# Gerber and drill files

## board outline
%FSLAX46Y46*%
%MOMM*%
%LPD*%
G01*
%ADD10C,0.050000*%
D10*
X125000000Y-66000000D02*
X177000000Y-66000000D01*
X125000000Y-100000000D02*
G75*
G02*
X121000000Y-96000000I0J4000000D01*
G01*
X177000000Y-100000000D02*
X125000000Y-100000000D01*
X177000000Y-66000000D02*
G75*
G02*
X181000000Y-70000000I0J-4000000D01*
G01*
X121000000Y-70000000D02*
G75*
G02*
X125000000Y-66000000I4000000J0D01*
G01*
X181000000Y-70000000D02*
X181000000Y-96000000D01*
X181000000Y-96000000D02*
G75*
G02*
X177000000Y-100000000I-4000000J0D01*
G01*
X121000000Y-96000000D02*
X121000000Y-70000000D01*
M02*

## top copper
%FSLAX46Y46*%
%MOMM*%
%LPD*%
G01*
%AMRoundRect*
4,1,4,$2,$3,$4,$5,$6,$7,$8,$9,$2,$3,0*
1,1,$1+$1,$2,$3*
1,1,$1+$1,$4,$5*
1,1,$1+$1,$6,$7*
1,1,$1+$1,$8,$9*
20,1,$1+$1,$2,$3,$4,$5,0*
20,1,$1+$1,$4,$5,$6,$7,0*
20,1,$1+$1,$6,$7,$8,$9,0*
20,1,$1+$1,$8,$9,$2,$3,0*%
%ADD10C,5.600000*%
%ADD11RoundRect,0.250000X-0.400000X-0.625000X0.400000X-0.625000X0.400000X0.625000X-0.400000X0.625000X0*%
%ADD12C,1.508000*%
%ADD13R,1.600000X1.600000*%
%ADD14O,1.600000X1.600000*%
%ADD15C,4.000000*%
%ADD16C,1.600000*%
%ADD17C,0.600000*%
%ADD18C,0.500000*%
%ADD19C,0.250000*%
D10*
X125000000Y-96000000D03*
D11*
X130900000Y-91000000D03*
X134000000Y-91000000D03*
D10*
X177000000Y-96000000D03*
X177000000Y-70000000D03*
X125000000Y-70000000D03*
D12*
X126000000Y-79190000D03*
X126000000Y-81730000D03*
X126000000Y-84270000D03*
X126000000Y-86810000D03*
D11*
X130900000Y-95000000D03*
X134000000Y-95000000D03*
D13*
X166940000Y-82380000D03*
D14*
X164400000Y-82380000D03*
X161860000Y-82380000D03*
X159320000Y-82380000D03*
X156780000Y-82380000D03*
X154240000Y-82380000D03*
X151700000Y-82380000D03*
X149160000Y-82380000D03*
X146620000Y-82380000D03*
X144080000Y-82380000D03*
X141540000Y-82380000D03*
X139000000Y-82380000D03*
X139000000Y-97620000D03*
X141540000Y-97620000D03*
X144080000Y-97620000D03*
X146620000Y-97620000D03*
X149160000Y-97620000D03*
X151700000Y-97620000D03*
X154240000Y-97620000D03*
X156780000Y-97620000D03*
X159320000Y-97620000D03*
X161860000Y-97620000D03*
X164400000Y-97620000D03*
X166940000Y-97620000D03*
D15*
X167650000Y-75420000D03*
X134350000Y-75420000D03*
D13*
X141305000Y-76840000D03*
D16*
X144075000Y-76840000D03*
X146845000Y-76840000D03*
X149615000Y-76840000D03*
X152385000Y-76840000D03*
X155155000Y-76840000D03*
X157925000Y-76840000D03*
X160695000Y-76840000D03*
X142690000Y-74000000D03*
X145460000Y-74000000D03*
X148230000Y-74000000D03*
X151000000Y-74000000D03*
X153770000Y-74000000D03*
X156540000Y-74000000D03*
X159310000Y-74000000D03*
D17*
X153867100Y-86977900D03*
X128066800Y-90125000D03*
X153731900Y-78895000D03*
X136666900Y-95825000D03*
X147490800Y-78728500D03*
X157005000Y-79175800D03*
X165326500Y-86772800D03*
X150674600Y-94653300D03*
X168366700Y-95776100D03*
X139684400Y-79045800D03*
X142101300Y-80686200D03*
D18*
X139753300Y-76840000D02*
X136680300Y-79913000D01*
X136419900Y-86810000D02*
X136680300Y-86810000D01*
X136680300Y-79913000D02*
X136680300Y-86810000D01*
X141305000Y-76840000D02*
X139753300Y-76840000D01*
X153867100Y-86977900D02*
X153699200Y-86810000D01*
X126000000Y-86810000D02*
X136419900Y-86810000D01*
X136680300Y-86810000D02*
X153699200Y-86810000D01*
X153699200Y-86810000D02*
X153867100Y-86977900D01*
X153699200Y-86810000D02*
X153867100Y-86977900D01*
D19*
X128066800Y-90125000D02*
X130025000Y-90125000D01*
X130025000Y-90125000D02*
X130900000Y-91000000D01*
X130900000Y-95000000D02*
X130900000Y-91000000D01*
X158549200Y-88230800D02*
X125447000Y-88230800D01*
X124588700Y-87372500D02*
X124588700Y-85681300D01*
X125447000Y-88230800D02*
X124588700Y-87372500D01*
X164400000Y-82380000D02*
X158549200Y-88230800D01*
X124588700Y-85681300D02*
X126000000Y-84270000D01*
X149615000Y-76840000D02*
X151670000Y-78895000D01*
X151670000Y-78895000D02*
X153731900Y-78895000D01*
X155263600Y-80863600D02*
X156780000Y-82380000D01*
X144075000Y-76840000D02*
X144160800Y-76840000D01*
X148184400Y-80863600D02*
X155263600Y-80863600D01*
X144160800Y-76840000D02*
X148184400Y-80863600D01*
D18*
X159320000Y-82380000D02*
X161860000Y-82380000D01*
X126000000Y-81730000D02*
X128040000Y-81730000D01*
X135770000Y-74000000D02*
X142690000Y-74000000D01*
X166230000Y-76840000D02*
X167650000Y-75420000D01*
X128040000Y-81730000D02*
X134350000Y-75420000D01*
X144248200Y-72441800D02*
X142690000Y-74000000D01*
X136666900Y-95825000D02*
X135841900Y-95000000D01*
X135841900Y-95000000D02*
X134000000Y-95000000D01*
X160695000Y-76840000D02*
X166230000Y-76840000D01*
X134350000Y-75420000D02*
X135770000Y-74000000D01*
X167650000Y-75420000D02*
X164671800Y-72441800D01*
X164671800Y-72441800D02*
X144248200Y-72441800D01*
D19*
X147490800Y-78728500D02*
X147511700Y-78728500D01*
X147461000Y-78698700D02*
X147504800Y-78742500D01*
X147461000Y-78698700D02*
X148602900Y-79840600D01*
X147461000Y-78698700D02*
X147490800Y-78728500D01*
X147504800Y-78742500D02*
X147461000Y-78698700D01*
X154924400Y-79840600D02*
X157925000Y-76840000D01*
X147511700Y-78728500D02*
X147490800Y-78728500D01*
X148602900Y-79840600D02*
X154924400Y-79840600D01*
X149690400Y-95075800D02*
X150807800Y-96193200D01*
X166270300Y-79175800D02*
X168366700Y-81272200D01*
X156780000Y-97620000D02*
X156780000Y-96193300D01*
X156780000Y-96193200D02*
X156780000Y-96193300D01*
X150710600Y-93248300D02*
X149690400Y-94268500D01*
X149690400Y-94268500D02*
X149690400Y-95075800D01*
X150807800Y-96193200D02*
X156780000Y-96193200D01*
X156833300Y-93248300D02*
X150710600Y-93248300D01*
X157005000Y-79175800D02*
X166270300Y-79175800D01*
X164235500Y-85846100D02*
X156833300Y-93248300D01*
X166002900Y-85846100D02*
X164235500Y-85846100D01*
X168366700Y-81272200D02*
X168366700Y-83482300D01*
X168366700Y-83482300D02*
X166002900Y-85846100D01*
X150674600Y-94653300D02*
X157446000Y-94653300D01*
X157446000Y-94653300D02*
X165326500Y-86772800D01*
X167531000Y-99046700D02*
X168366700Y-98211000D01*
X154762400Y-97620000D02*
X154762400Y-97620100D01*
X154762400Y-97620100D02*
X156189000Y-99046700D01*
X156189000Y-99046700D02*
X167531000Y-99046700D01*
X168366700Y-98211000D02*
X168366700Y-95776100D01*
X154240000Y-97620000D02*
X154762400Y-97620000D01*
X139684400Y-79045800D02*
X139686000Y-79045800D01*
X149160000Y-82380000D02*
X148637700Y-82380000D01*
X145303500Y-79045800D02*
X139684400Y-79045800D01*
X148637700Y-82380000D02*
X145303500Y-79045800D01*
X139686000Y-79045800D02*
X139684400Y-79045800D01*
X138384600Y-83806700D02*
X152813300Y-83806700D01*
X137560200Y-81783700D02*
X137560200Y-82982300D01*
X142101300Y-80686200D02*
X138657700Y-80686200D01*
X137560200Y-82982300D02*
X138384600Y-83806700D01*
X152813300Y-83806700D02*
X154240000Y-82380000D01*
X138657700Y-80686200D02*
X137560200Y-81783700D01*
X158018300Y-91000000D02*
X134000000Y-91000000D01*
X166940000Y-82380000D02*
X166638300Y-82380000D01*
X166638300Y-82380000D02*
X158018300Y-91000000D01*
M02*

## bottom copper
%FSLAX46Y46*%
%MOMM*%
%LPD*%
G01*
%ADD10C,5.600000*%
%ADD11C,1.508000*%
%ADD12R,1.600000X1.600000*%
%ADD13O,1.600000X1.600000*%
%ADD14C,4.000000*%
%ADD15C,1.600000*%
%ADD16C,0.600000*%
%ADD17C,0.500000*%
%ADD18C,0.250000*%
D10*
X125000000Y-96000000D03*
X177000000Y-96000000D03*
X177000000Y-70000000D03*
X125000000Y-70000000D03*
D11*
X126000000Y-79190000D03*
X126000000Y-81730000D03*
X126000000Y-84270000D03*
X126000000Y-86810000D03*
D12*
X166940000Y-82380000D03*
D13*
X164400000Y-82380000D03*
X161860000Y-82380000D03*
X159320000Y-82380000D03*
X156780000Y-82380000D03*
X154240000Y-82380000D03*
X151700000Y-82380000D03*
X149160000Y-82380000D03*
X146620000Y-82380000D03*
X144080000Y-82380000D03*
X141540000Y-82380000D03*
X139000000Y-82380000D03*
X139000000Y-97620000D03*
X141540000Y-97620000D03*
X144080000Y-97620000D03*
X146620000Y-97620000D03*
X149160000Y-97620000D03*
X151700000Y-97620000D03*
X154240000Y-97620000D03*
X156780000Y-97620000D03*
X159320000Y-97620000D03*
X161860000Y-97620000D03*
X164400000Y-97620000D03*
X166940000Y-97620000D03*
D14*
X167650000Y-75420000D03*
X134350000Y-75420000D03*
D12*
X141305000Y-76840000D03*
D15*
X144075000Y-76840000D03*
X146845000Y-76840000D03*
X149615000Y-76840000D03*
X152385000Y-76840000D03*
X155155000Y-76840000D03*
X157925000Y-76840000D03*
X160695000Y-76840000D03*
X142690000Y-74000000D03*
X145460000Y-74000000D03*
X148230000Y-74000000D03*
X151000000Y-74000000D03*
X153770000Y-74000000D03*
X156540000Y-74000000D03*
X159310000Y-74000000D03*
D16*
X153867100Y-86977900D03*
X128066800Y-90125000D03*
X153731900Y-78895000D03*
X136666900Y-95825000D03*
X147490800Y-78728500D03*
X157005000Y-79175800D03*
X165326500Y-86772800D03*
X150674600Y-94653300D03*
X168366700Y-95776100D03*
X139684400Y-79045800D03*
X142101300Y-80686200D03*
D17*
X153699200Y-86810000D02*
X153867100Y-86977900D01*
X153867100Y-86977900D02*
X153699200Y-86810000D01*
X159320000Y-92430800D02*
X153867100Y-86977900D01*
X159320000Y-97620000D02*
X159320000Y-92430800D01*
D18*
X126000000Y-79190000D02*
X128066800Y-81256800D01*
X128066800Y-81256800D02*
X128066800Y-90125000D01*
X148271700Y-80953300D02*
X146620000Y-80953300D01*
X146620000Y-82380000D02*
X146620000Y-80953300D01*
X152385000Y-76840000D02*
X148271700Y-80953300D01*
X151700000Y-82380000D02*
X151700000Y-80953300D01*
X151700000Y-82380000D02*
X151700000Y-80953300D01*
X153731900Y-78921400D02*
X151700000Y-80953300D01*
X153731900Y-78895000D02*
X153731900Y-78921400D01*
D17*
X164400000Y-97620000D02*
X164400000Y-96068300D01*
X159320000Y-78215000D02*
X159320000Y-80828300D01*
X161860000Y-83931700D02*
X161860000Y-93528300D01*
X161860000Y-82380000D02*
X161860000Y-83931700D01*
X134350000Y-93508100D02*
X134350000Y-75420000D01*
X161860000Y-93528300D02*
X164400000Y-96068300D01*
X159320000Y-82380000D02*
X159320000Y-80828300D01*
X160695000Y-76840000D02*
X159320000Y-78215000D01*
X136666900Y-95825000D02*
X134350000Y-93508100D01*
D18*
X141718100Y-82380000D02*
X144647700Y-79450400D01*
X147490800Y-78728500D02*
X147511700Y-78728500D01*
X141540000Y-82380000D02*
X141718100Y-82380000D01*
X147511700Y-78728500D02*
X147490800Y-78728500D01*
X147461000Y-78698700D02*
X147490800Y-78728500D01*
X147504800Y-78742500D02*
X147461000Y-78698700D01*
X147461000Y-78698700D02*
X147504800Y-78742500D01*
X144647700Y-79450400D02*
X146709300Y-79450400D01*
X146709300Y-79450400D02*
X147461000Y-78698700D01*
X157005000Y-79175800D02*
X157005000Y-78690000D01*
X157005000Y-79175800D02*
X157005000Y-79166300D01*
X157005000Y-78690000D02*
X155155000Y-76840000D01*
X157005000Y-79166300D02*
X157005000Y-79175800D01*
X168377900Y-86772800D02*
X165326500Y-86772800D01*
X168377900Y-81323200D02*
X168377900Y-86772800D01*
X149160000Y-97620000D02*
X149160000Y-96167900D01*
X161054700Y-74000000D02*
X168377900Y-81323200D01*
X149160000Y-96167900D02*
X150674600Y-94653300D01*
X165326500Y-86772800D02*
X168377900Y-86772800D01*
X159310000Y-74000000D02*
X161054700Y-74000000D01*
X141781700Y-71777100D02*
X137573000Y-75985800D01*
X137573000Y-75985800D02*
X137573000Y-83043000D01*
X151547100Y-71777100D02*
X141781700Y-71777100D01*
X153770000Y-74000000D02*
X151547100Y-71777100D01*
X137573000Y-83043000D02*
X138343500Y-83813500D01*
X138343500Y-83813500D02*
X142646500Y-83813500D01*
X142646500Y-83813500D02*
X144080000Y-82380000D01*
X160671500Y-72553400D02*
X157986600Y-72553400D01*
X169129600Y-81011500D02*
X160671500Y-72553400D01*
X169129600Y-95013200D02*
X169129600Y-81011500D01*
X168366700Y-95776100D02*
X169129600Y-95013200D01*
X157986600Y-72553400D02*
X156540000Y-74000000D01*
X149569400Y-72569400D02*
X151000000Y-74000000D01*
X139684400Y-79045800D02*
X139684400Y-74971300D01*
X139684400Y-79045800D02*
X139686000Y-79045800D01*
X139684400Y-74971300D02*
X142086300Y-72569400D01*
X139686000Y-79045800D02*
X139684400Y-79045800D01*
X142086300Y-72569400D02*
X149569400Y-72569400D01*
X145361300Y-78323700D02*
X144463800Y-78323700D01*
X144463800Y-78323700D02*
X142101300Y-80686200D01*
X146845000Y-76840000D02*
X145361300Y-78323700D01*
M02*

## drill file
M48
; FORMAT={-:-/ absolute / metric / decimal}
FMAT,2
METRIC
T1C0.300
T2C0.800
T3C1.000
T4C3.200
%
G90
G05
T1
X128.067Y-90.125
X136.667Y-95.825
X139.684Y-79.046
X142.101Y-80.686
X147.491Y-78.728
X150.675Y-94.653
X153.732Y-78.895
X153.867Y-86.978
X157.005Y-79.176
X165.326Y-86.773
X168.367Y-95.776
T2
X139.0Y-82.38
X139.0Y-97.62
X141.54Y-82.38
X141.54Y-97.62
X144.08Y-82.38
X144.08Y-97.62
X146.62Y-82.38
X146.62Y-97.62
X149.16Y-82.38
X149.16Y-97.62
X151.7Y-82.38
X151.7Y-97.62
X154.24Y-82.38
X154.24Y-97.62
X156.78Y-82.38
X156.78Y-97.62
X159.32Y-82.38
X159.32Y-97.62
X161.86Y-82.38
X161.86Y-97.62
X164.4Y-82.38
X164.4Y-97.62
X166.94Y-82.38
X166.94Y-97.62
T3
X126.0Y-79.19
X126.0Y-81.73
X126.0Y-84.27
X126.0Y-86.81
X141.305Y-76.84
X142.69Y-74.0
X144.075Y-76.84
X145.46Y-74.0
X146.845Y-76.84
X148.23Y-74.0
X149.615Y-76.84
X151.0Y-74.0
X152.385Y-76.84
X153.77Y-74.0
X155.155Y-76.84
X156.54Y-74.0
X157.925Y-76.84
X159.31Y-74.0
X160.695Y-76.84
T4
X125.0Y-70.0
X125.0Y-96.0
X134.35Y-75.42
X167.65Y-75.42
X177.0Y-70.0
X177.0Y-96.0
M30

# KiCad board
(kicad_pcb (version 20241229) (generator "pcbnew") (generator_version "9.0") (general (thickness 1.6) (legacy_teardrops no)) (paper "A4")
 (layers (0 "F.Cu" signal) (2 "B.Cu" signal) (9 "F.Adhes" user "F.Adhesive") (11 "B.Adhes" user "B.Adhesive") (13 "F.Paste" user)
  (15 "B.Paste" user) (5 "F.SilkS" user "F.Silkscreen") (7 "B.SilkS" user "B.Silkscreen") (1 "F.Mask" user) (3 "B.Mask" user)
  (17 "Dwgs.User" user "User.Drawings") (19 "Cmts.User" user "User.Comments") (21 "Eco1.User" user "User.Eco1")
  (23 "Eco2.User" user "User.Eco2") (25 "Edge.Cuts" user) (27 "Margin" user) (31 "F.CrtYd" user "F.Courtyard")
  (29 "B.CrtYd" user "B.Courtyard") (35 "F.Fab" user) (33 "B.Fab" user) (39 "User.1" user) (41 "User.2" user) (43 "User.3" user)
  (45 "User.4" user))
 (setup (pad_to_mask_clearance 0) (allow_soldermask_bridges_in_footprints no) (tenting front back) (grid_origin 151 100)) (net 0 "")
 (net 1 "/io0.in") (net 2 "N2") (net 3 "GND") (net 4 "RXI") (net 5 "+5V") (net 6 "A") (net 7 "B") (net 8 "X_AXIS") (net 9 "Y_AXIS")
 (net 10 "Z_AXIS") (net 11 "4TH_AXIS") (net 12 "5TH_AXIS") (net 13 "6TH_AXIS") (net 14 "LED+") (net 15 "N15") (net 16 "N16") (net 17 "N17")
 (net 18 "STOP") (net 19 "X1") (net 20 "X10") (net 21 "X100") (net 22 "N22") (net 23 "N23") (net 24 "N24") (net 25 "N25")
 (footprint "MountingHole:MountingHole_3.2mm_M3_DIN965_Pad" (layer "F.Cu") (at 125 96)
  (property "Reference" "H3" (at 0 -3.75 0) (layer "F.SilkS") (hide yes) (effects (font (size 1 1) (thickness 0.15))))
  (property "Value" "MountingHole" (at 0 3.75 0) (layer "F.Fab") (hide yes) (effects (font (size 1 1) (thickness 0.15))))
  (pad "1" thru_hole circle (at 0 0) (size 5.6 5.6) (drill 3.2) (layers "*.Cu" "*.Mask") (remove_unused_layers no) (zone_connect 2)))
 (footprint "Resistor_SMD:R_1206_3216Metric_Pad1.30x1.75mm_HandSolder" (layer "F.Cu") (at 132.45 91)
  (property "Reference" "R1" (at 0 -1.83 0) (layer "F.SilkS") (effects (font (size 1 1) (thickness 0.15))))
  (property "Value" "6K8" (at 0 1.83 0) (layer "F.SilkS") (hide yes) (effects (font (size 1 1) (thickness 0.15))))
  (pad "1" smd roundrect (at -1.55 0) (size 1.3 1.75) (layers "F.Cu" "F.Mask" "F.Paste") (roundrect_rratio 0.192308) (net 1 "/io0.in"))
  (pad "2" smd roundrect (at 1.55 0) (size 1.3 1.75) (layers "F.Cu" "F.Mask" "F.Paste") (roundrect_rratio 0.192308) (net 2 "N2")))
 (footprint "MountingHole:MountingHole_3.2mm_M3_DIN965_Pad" (layer "F.Cu") (at 177 96)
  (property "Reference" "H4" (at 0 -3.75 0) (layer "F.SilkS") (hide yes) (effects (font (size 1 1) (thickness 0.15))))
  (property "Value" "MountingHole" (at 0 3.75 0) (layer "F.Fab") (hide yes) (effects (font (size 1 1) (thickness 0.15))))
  (pad "1" thru_hole circle (at 0 0) (size 5.6 5.6) (drill 3.2) (layers "*.Cu" "*.Mask") (remove_unused_layers no) (zone_connect 2)))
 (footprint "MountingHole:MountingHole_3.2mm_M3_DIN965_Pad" (layer "F.Cu") (at 177 70)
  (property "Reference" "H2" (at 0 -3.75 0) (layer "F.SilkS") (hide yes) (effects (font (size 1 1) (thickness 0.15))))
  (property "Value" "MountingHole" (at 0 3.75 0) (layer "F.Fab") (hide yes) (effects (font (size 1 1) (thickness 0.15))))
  (pad "1" thru_hole circle (at 0 0) (size 5.6 5.6) (drill 3.2) (layers "*.Cu" "*.Mask") (remove_unused_layers no) (zone_connect 2)))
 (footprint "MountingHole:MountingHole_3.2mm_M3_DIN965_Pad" (layer "F.Cu") (at 125 70)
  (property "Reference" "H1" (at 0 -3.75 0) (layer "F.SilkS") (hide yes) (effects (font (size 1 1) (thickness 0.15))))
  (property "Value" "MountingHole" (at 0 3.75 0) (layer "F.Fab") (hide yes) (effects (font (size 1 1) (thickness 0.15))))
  (pad "1" thru_hole circle (at 0 0) (size 5.6 5.6) (drill 3.2) (layers "*.Cu" "*.Mask") (remove_unused_layers no) (zone_connect 2)))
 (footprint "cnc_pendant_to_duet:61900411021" (layer "F.Cu") (at 122.65 83 -90)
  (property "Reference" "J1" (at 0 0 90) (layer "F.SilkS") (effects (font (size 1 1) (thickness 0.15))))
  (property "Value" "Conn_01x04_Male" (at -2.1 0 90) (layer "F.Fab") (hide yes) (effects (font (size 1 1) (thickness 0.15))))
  (pad "1" thru_hole circle (at -3.81 -3.35 270) (size 1.508 1.508) (drill 1) (layers "*.Cu" "*.Mask") (remove_unused_layers no)
   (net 1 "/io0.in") (solder_mask_margin 0.102))
  (pad "2" thru_hole circle (at -1.27 -3.35 270) (size 1.508 1.508) (drill 1) (layers "*.Cu" "*.Mask") (remove_unused_layers no)
   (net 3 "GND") (solder_mask_margin 0.102))
  (pad "3" thru_hole circle (at 1.27 -3.35 270) (size 1.508 1.508) (drill 1) (layers "*.Cu" "*.Mask") (remove_unused_layers no)
   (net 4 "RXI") (solder_mask_margin 0.102))
  (pad "4" thru_hole circle (at 3.81 -3.35 270) (size 1.508 1.508) (drill 1) (layers "*.Cu" "*.Mask") (remove_unused_layers no)
   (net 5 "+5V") (solder_mask_margin 0.102)))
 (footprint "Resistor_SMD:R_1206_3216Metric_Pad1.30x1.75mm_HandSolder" (layer "F.Cu") (at 132.45 95)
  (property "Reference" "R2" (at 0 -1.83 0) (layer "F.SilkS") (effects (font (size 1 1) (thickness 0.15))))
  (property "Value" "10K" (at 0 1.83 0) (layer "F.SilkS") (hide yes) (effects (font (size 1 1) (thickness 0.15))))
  (pad "1" smd roundrect (at -1.55 0) (size 1.3 1.75) (layers "F.Cu" "F.Mask" "F.Paste") (roundrect_rratio 0.192308) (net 1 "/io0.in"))
  (pad "2" smd roundrect (at 1.55 0) (size 1.3 1.75) (layers "F.Cu" "F.Mask" "F.Paste") (roundrect_rratio 0.192308) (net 3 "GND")))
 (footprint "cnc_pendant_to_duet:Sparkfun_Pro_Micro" (layer "F.Cu") (at 139 97.62 90)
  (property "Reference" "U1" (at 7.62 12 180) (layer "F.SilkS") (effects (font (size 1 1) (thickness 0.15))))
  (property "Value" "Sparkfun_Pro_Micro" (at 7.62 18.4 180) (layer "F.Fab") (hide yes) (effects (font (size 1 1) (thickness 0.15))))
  (pad "1" thru_hole rect (at 15.24 27.94 90) (size 1.6 1.6) (drill 0.8) (layers "*.Cu" "*.Mask") (remove_unused_layers no) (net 2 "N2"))
  (pad "2" thru_hole oval (at 15.24 25.4 90) (size 1.6 1.6) (drill 0.8) (layers "*.Cu" "*.Mask") (remove_unused_layers no) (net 4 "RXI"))
  (pad "3" thru_hole oval (at 15.24 22.86 90) (size 1.6 1.6) (drill 0.8) (layers "*.Cu" "*.Mask") (remove_unused_layers no) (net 3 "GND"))
  (pad "4" thru_hole oval (at 15.24 20.32 90) (size 1.6 1.6) (drill 0.8) (layers "*.Cu" "*.Mask") (remove_unused_layers no) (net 3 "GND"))
  (pad "5" thru_hole oval (at 15.24 17.78 90) (size 1.6 1.6) (drill 0.8) (layers "*.Cu" "*.Mask") (remove_unused_layers no) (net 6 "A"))
  (pad "6" thru_hole oval (at 15.24 15.24 90) (size 1.6 1.6) (drill 0.8) (layers "*.Cu" "*.Mask") (remove_unused_layers no) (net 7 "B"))
  (pad "7" thru_hole oval (at 15.24 12.7 90) (size 1.6 1.6) (drill 0.8) (layers "*.Cu" "*.Mask") (remove_unused_layers no) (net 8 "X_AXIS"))
  (pad "8" thru_hole oval (at 15.24 10.16 90) (size 1.6 1.6) (drill 0.8) (layers "*.Cu" "*.Mask") (remove_unused_layers no) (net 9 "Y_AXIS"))
  (pad "9" thru_hole oval (at 15.24 7.62 90) (size 1.6 1.6) (drill 0.8) (layers "*.Cu" "*.Mask") (remove_unused_layers no) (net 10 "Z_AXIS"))
  (pad "10" thru_hole oval (at 15.24 5.08 90) (size 1.6 1.6) (drill 0.8) (layers "*.Cu" "*.Mask") (remove_unused_layers no)
   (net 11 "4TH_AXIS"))
  (pad "11" thru_hole oval (at 15.24 2.54 90) (size 1.6 1.6) (drill 0.8) (layers "*.Cu" "*.Mask") (remove_unused_layers no)
   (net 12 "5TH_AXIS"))
  (pad "12" thru_hole oval (at 15.24 0 90) (size 1.6 1.6) (drill 0.8) (layers "*.Cu" "*.Mask") (remove_unused_layers no) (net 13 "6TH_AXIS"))
  (pad "13" thru_hole oval (at 0 0 90) (size 1.6 1.6) (drill 0.8) (layers "*.Cu" "*.Mask") (remove_unused_layers no) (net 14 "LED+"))
  (pad "14" thru_hole oval (at 0 2.54 90) (size 1.6 1.6) (drill 0.8) (layers "*.Cu" "*.Mask") (remove_unused_layers no) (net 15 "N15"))
  (pad "15" thru_hole oval (at 0 5.08 90) (size 1.6 1.6) (drill 0.8) (layers "*.Cu" "*.Mask") (remove_unused_layers no) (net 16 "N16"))
  (pad "16" thru_hole oval (at 0 7.62 90) (size 1.6 1.6) (drill 0.8) (layers "*.Cu" "*.Mask") (remove_unused_layers no) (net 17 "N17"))
  (pad "17" thru_hole oval (at 0 10.16 90) (size 1.6 1.6) (drill 0.8) (layers "*.Cu" "*.Mask") (remove_unused_layers no) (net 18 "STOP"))
  (pad "18" thru_hole oval (at 0 12.7 90) (size 1.6 1.6) (drill 0.8) (layers "*.Cu" "*.Mask") (remove_unused_layers no) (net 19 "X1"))
  (pad "19" thru_hole oval (at 0 15.24 90) (size 1.6 1.6) (drill 0.8) (layers "*.Cu" "*.Mask") (remove_unused_layers no) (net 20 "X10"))
  (pad "20" thru_hole oval (at 0 17.78 90) (size 1.6 1.6) (drill 0.8) (layers "*.Cu" "*.Mask") (remove_unused_layers no) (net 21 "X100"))
  (pad "21" thru_hole oval (at 0 20.32 90) (size 1.6 1.6) (drill 0.8) (layers "*.Cu" "*.Mask") (remove_unused_layers no) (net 5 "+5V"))
  (pad "22" thru_hole oval (at 0 22.86 90) (size 1.6 1.6) (drill 0.8) (layers "*.Cu" "*.Mask") (remove_unused_layers no) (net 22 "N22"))
  (pad "23" thru_hole oval (at 0 25.4 90) (size 1.6 1.6) (drill 0.8) (layers "*.Cu" "*.Mask") (remove_unused_layers no) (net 3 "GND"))
  (pad "24" thru_hole oval (at 0 27.94 90) (size 1.6 1.6) (drill 0.8) (layers "*.Cu" "*.Mask") (remove_unused_layers no) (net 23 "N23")))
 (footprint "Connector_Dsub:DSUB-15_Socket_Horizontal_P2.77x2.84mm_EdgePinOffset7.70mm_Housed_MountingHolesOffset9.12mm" (layer "F.Cu")
  (at 141.305 76.84 180)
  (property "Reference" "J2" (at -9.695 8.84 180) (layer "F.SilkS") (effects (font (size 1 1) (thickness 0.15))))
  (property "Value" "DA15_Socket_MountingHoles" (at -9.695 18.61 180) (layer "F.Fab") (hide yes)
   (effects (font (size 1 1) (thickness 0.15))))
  (pad "0" thru_hole circle (at -26.345 1.42 180) (size 4 4) (drill 3.2) (layers "*.Cu" "*.Mask") (remove_unused_layers no) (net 3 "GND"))
  (pad "0" thru_hole circle (at 6.955 1.42 180) (size 4 4) (drill 3.2) (layers "*.Cu" "*.Mask") (remove_unused_layers no) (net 3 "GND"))
  (pad "1" thru_hole rect (at 0 0 180) (size 1.6 1.6) (drill 1) (layers "*.Cu" "*.Mask") (remove_unused_layers no) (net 5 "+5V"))
  (pad "2" thru_hole circle (at -2.77 0 180) (size 1.6 1.6) (drill 1) (layers "*.Cu" "*.Mask") (remove_unused_layers no) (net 6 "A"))
  (pad "3" thru_hole circle (at -5.54 0 180) (size 1.6 1.6) (drill 1) (layers "*.Cu" "*.Mask") (remove_unused_layers no) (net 7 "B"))
  (pad "4" thru_hole circle (at -8.31 0 180) (size 1.6 1.6) (drill 1) (layers "*.Cu" "*.Mask") (remove_unused_layers no) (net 8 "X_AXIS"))
  (pad "5" thru_hole circle (at -11.08 0 180) (size 1.6 1.6) (drill 1) (layers "*.Cu" "*.Mask") (remove_unused_layers no) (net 10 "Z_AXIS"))
  (pad "6" thru_hole circle (at -13.85 0 180) (size 1.6 1.6) (drill 1) (layers "*.Cu" "*.Mask") (remove_unused_layers no) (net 21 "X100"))
  (pad "7" thru_hole circle (at -16.62 0 180) (size 1.6 1.6) (drill 1) (layers "*.Cu" "*.Mask") (remove_unused_layers no)
   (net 12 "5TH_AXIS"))
  (pad "8" thru_hole circle (at -19.39 0 180) (size 1.6 1.6) (drill 1) (layers "*.Cu" "*.Mask") (remove_unused_layers no) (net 3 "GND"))
  (pad "9" thru_hole circle (at -1.385 2.84 180) (size 1.6 1.6) (drill 1) (layers "*.Cu" "*.Mask") (remove_unused_layers no) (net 3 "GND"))
  (pad "10" thru_hole circle (at -4.155 2.84 180) (size 1.6 1.6) (drill 1) (layers "*.Cu" "*.Mask") (remove_unused_layers no) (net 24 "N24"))
  (pad "11" thru_hole circle (at -6.925 2.84 180) (size 1.6 1.6) (drill 1) (layers "*.Cu" "*.Mask") (remove_unused_layers no) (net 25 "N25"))
  (pad "12" thru_hole circle (at -9.695 2.84 180) (size 1.6 1.6) (drill 1) (layers "*.Cu" "*.Mask") (remove_unused_layers no)
   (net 9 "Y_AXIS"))
  (pad "13" thru_hole circle (at -12.465 2.84 180) (size 1.6 1.6) (drill 1) (layers "*.Cu" "*.Mask") (remove_unused_layers no)
   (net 11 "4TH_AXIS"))
  (pad "14" thru_hole circle (at -15.235 2.84 180) (size 1.6 1.6) (drill 1) (layers "*.Cu" "*.Mask") (remove_unused_layers no)
   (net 20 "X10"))
  (pad "15" thru_hole circle (at -18.005 2.84 180) (size 1.6 1.6) (drill 1) (layers "*.Cu" "*.Mask") (remove_unused_layers no)
   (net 18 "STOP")))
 (gr_line (start 125 66) (end 177 66) (stroke (width 0.05) (type default)) (layer "Edge.Cuts"))
 (gr_arc (start 125 100) (mid 122.171573 98.828427) (end 121 96) (stroke (width 0.05) (type default)) (layer "Edge.Cuts"))
 (gr_line (start 177 100) (end 125 100) (stroke (width 0.05) (type default)) (layer "Edge.Cuts"))
 (gr_arc (start 177 66) (mid 179.828427 67.171573) (end 181 70) (stroke (width 0.05) (type default)) (layer "Edge.Cuts"))
 (gr_arc (start 121 70) (mid 122.171573 67.171573) (end 125 66) (stroke (width 0.05) (type default)) (layer "Edge.Cuts"))
 (gr_line (start 181 70) (end 181 96) (stroke (width 0.05) (type default)) (layer "Edge.Cuts"))
 (gr_arc (start 181 96) (mid 179.828427 98.828427) (end 177 100) (stroke (width 0.05) (type default)) (layer "Edge.Cuts"))
 (gr_line (start 121 96) (end 121 70) (stroke (width 0.05) (type default)) (layer "Edge.Cuts"))
 (segment (start 139.7533 76.84) (end 136.6803 79.913) (width 0.5) (layer "F.Cu") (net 5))
 (segment (start 136.4199 86.81) (end 136.6803 86.81) (width 0.5) (layer "F.Cu") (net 5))
 (segment (start 136.6803 79.913) (end 136.6803 86.81) (width 0.5) (layer "F.Cu") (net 5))
 (segment (start 141.305 76.84) (end 139.7533 76.84) (width 0.5) (layer "F.Cu") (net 5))
 (segment (start 153.8671 86.9779) (end 153.6992 86.81) (width 0.5) (layer "F.Cu") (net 5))
 (segment (start 126 86.81) (end 136.4199 86.81) (width 0.5) (layer "F.Cu") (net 5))
 (segment (start 136.6803 86.81) (end 153.6992 86.81) (width 0.5) (layer "F.Cu") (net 5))
 (segment (start 153.6992 86.81) (end 153.8671 86.9779) (width 0.5) (layer "F.Cu") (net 5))
 (segment (start 153.6992 86.81) (end 153.8671 86.9779) (width 0.5) (layer "F.Cu") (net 5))
 (via (at 153.8671 86.9779) (size 0.6) (drill 0.3) (layers "F.Cu" "B.Cu") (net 5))
 (segment (start 153.6992 86.81) (end 153.8671 86.9779) (width 0.5) (layer "B.Cu") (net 5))
 (segment (start 153.8671 86.9779) (end 153.6992 86.81) (width 0.5) (layer "B.Cu") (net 5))
 (segment (start 159.32 92.4308) (end 153.8671 86.9779) (width 0.5) (layer "B.Cu") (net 5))
 (segment (start 159.32 97.62) (end 159.32 92.4308) (width 0.5) (layer "B.Cu") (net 5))
 (segment (start 128.0668 90.125) (end 130.025 90.125) (width 0.25) (layer "F.Cu") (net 1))
 (segment (start 130.025 90.125) (end 130.9 91) (width 0.25) (layer "F.Cu") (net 1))
 (segment (start 130.9 95) (end 130.9 91) (width 0.25) (layer "F.Cu") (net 1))
 (via (at 128.0668 90.125) (size 0.6) (drill 0.3) (layers "F.Cu" "B.Cu") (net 1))
 (segment (start 126 79.19) (end 128.0668 81.2568) (width 0.25) (layer "B.Cu") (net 1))
 (segment (start 128.0668 81.2568) (end 128.0668 90.125) (width 0.25) (layer "B.Cu") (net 1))
 (segment (start 158.5492 88.2308) (end 125.447 88.2308) (width 0.25) (layer "F.Cu") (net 4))
 (segment (start 124.5887 87.3725) (end 124.5887 85.6813) (width 0.25) (layer "F.Cu") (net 4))
 (segment (start 125.447 88.2308) (end 124.5887 87.3725) (width 0.25) (layer "F.Cu") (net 4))
 (segment (start 164.4 82.38) (end 158.5492 88.2308) (width 0.25) (layer "F.Cu") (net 4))
 (segment (start 124.5887 85.6813) (end 126 84.27) (width 0.25) (layer "F.Cu") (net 4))
 (segment (start 148.2717 80.9533) (end 146.62 80.9533) (width 0.25) (layer "B.Cu") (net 10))
 (segment (start 146.62 82.38) (end 146.62 80.9533) (width 0.25) (layer "B.Cu") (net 10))
 (segment (start 152.385 76.84) (end 148.2717 80.9533) (width 0.25) (layer "B.Cu") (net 10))
 (segment (start 149.615 76.84) (end 151.67 78.895) (width 0.25) (layer "F.Cu") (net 8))
 (segment (start 151.67 78.895) (end 153.7319 78.895) (width 0.25) (layer "F.Cu") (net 8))
 (via (at 153.7319 78.895) (size 0.6) (drill 0.3) (layers "F.Cu" "B.Cu") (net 8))
 (segment (start 151.7 82.38) (end 151.7 80.9533) (width 0.25) (layer "B.Cu") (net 8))
 (segment (start 151.7 82.38) (end 151.7 80.9533) (width 0.25) (layer "B.Cu") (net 8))
 (segment (start 153.7319 78.9214) (end 151.7 80.9533) (width 0.25) (layer "B.Cu") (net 8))
 (segment (start 153.7319 78.895) (end 153.7319 78.9214) (width 0.25) (layer "B.Cu") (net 8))
 (segment (start 155.2636 80.8636) (end 156.78 82.38) (width 0.25) (layer "F.Cu") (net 6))
 (segment (start 144.075 76.84) (end 144.1608 76.84) (width 0.25) (layer "F.Cu") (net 6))
 (segment (start 148.1844 80.8636) (end 155.2636 80.8636) (width 0.25) (layer "F.Cu") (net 6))
 (segment (start 144.1608 76.84) (end 148.1844 80.8636) (width 0.25) (layer "F.Cu") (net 6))
 (segment (start 159.32 82.38) (end 161.86 82.38) (width 0.5) (layer "F.Cu") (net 3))
 (segment (start 126 81.73) (end 128.04 81.73) (width 0.5) (layer "F.Cu") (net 3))
 (segment (start 135.77 74) (end 142.69 74) (width 0.5) (layer "F.Cu") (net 3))
 (segment (start 166.23 76.84) (end 167.65 75.42) (width 0.5) (layer "F.Cu") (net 3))
 (segment (start 128.04 81.73) (end 134.35 75.42) (width 0.5) (layer "F.Cu") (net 3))
 (segment (start 144.2482 72.4418) (end 142.69 74) (width 0.5) (layer "F.Cu") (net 3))
 (segment (start 136.6669 95.825) (end 135.8419 95) (width 0.5) (layer "F.Cu") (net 3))
 (segment (start 135.8419 95) (end 134 95) (width 0.5) (layer "F.Cu") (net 3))
 (segment (start 160.695 76.84) (end 166.23 76.84) (width 0.5) (layer "F.Cu") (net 3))
 (segment (start 134.35 75.42) (end 135.77 74) (width 0.5) (layer "F.Cu") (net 3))
 (segment (start 167.65 75.42) (end 164.6718 72.4418) (width 0.5) (layer "F.Cu") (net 3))
 (segment (start 164.6718 72.4418) (end 144.2482 72.4418) (width 0.5) (layer "F.Cu") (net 3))
 (via (at 136.6669 95.825) (size 0.6) (drill 0.3) (layers "F.Cu" "B.Cu") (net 3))
 (segment (start 164.4 97.62) (end 164.4 96.0683) (width 0.5) (layer "B.Cu") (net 3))
 (segment (start 159.32 78.215) (end 159.32 80.8283) (width 0.5) (layer "B.Cu") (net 3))
 (segment (start 161.86 83.9317) (end 161.86 93.5283) (width 0.5) (layer "B.Cu") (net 3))
 (segment (start 161.86 82.38) (end 161.86 83.9317) (width 0.5) (layer "B.Cu") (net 3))
 (segment (start 134.35 93.5081) (end 134.35 75.42) (width 0.5) (layer "B.Cu") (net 3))
 (segment (start 161.86 93.5283) (end 164.4 96.0683) (width 0.5) (layer "B.Cu") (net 3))
 (segment (start 159.32 82.38) (end 159.32 80.8283) (width 0.5) (layer "B.Cu") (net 3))
 (segment (start 160.695 76.84) (end 159.32 78.215) (width 0.5) (layer "B.Cu") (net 3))
 (segment (start 136.6669 95.825) (end 134.35 93.5081) (width 0.5) (layer "B.Cu") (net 3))
 (segment (start 147.4908 78.7285) (end 147.5117 78.7285) (width 0.25) (layer "F.Cu") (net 12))
 (segment (start 147.461 78.6987) (end 147.5048 78.7425) (width 0.25) (layer "F.Cu") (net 12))
 (segment (start 147.461 78.6987) (end 148.6029 79.8406) (width 0.25) (layer "F.Cu") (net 12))
 (segment (start 147.461 78.6987) (end 147.4908 78.7285) (width 0.25) (layer "F.Cu") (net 12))
 (segment (start 147.5048 78.7425) (end 147.461 78.6987) (width 0.25) (layer "F.Cu") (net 12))
 (segment (start 154.9244 79.8406) (end 157.925 76.84) (width 0.25) (layer "F.Cu") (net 12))
 (segment (start 147.5117 78.7285) (end 147.4908 78.7285) (width 0.25) (layer "F.Cu") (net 12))
 (segment (start 148.6029 79.8406) (end 154.9244 79.8406) (width 0.25) (layer "F.Cu") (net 12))
 (via (at 147.4908 78.7285) (size 0.6) (drill 0.3) (layers "F.Cu" "B.Cu") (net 12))
 (segment (start 141.7181 82.38) (end 144.6477 79.4504) (width 0.25) (layer "B.Cu") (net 12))
 (segment (start 147.4908 78.7285) (end 147.5117 78.7285) (width 0.25) (layer "B.Cu") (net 12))
 (segment (start 141.54 82.38) (end 141.7181 82.38) (width 0.25) (layer "B.Cu") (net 12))
 (segment (start 147.5117 78.7285) (end 147.4908 78.7285) (width 0.25) (layer "B.Cu") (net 12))
 (segment (start 147.461 78.6987) (end 147.4908 78.7285) (width 0.25) (layer "B.Cu") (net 12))
 (segment (start 147.5048 78.7425) (end 147.461 78.6987) (width 0.25) (layer "B.Cu") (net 12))
 (segment (start 147.461 78.6987) (end 147.5048 78.7425) (width 0.25) (layer "B.Cu") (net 12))
 (segment (start 144.6477 79.4504) (end 146.7093 79.4504) (width 0.25) (layer "B.Cu") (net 12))
 (segment (start 146.7093 79.4504) (end 147.461 78.6987) (width 0.25) (layer "B.Cu") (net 12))
 (segment (start 149.6904 95.0758) (end 150.8078 96.1932) (width 0.25) (layer "F.Cu") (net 21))
 (segment (start 166.2703 79.1758) (end 168.3667 81.2722) (width 0.25) (layer "F.Cu") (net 21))
 (segment (start 156.78 97.62) (end 156.78 96.1933) (width 0.25) (layer "F.Cu") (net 21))
 (segment (start 156.78 96.1932) (end 156.78 96.1933) (width 0.25) (layer "F.Cu") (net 21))
 (segment (start 150.7106 93.2483) (end 149.6904 94.2685) (width 0.25) (layer "F.Cu") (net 21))
 (segment (start 149.6904 94.2685) (end 149.6904 95.0758) (width 0.25) (layer "F.Cu") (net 21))
 (segment (start 150.8078 96.1932) (end 156.78 96.1932) (width 0.25) (layer "F.Cu") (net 21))
 (segment (start 156.8333 93.2483) (end 150.7106 93.2483) (width 0.25) (layer "F.Cu") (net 21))
 (segment (start 157.005 79.1758) (end 166.2703 79.1758) (width 0.25) (layer "F.Cu") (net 21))
 (segment (start 164.2355 85.8461) (end 156.8333 93.2483) (width 0.25) (layer "F.Cu") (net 21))
 (segment (start 166.0029 85.8461) (end 164.2355 85.8461) (width 0.25) (layer "F.Cu") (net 21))
 (segment (start 168.3667 81.2722) (end 168.3667 83.4823) (width 0.25) (layer "F.Cu") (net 21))
 (segment (start 168.3667 83.4823) (end 166.0029 85.8461) (width 0.25) (layer "F.Cu") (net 21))
 (via (at 157.005 79.1758) (size 0.6) (drill 0.3) (layers "F.Cu" "B.Cu") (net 21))
 (segment (start 157.005 79.1758) (end 157.005 78.69) (width 0.25) (layer "B.Cu") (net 21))
 (segment (start 157.005 79.1758) (end 157.005 79.1663) (width 0.25) (layer "B.Cu") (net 21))
 (segment (start 157.005 78.69) (end 155.155 76.84) (width 0.25) (layer "B.Cu") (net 21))
 (segment (start 157.005 79.1663) (end 157.005 79.1758) (width 0.25) (layer "B.Cu") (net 21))
 (segment (start 150.6746 94.6533) (end 157.446 94.6533) (width 0.25) (layer "F.Cu") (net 18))
 (segment (start 157.446 94.6533) (end 165.3265 86.7728) (width 0.25) (layer "F.Cu") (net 18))
 (via (at 165.3265 86.7728) (size 0.6) (drill 0.3) (layers "F.Cu" "B.Cu") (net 18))
 (via (at 150.6746 94.6533) (size 0.6) (drill 0.3) (layers "F.Cu" "B.Cu") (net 18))
 (segment (start 168.3779 86.7728) (end 165.3265 86.7728) (width 0.25) (layer "B.Cu") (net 18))
 (segment (start 168.3779 81.3232) (end 168.3779 86.7728) (width 0.25) (layer "B.Cu") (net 18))
 (segment (start 149.16 97.62) (end 149.16 96.1679) (width 0.25) (layer "B.Cu") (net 18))
 (segment (start 161.0547 74) (end 168.3779 81.3232) (width 0.25) (layer "B.Cu") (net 18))
 (segment (start 149.16 96.1679) (end 150.6746 94.6533) (width 0.25) (layer "B.Cu") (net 18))
 (segment (start 165.3265 86.7728) (end 168.3779 86.7728) (width 0.25) (layer "B.Cu") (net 18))
 (segment (start 159.31 74) (end 161.0547 74) (width 0.25) (layer "B.Cu") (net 18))
 (segment (start 141.7817 71.7771) (end 137.573 75.9858) (width 0.25) (layer "B.Cu") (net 11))
 (segment (start 137.573 75.9858) (end 137.573 83.043) (width 0.25) (layer "B.Cu") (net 11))
 (segment (start 151.5471 71.7771) (end 141.7817 71.7771) (width 0.25) (layer "B.Cu") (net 11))
 (segment (start 153.77 74) (end 151.5471 71.7771) (width 0.25) (layer "B.Cu") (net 11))
 (segment (start 137.573 83.043) (end 138.3435 83.8135) (width 0.25) (layer "B.Cu") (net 11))
 (segment (start 138.3435 83.8135) (end 142.6465 83.8135) (width 0.25) (layer "B.Cu") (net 11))
 (segment (start 142.6465 83.8135) (end 144.08 82.38) (width 0.25) (layer "B.Cu") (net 11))
 (segment (start 167.531 99.0467) (end 168.3667 98.211) (width 0.25) (layer "F.Cu") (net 20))
 (segment (start 154.7624 97.62) (end 154.7624 97.6201) (width 0.25) (layer "F.Cu") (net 20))
 (segment (start 154.7624 97.6201) (end 156.189 99.0467) (width 0.25) (layer "F.Cu") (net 20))
 (segment (start 156.189 99.0467) (end 167.531 99.0467) (width 0.25) (layer "F.Cu") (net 20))
 (segment (start 168.3667 98.211) (end 168.3667 95.7761) (width 0.25) (layer "F.Cu") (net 20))
 (segment (start 154.24 97.62) (end 154.7624 97.62) (width 0.25) (layer "F.Cu") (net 20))
 (via (at 168.3667 95.7761) (size 0.6) (drill 0.3) (layers "F.Cu" "B.Cu") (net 20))
 (segment (start 160.6715 72.5534) (end 157.9866 72.5534) (width 0.25) (layer "B.Cu") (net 20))
 (segment (start 169.1296 81.0115) (end 160.6715 72.5534) (width 0.25) (layer "B.Cu") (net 20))
 (segment (start 169.1296 95.0132) (end 169.1296 81.0115) (width 0.25) (layer "B.Cu") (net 20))
 (segment (start 168.3667 95.7761) (end 169.1296 95.0132) (width 0.25) (layer "B.Cu") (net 20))
 (segment (start 157.9866 72.5534) (end 156.54 74) (width 0.25) (layer "B.Cu") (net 20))
 (segment (start 139.6844 79.0458) (end 139.686 79.0458) (width 0.25) (layer "F.Cu") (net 9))
 (segment (start 149.16 82.38) (end 148.6377 82.38) (width 0.25) (layer "F.Cu") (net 9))
 (segment (start 145.3035 79.0458) (end 139.6844 79.0458) (width 0.25) (layer "F.Cu") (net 9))
 (segment (start 148.6377 82.38) (end 145.3035 79.0458) (width 0.25) (layer "F.Cu") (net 9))
 (segment (start 139.686 79.0458) (end 139.6844 79.0458) (width 0.25) (layer "F.Cu") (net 9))
 (via (at 139.6844 79.0458) (size 0.6) (drill 0.3) (layers "F.Cu" "B.Cu") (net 9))
 (segment (start 149.5694 72.5694) (end 151 74) (width 0.25) (layer "B.Cu") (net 9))
 (segment (start 139.6844 79.0458) (end 139.6844 74.9713) (width 0.25) (layer "B.Cu") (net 9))
 (segment (start 139.6844 79.0458) (end 139.686 79.0458) (width 0.25) (layer "B.Cu") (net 9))
 (segment (start 139.6844 74.9713) (end 142.0863 72.5694) (width 0.25) (layer "B.Cu") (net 9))
 (segment (start 139.686 79.0458) (end 139.6844 79.0458) (width 0.25) (layer "B.Cu") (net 9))
 (segment (start 142.0863 72.5694) (end 149.5694 72.5694) (width 0.25) (layer "B.Cu") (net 9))
 (segment (start 138.3846 83.8067) (end 152.8133 83.8067) (width 0.25) (layer "F.Cu") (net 7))
 (segment (start 137.5602 81.7837) (end 137.5602 82.9823) (width 0.25) (layer "F.Cu") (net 7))
 (segment (start 142.1013 80.6862) (end 138.6577 80.6862) (width 0.25) (layer "F.Cu") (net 7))
 (segment (start 137.5602 82.9823) (end 138.3846 83.8067) (width 0.25) (layer "F.Cu") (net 7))
 (segment (start 152.8133 83.8067) (end 154.24 82.38) (width 0.25) (layer "F.Cu") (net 7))
 (segment (start 138.6577 80.6862) (end 137.5602 81.7837) (width 0.25) (layer "F.Cu") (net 7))
 (via (at 142.1013 80.6862) (size 0.6) (drill 0.3) (layers "F.Cu" "B.Cu") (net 7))
 (segment (start 145.3613 78.3237) (end 144.4638 78.3237) (width 0.25) (layer "B.Cu") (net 7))
 (segment (start 144.4638 78.3237) (end 142.1013 80.6862) (width 0.25) (layer "B.Cu") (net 7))
 (segment (start 146.845 76.84) (end 145.3613 78.3237) (width 0.25) (layer "B.Cu") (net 7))
 (segment (start 158.0183 91) (end 134 91) (width 0.25) (layer "F.Cu") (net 2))
 (segment (start 166.94 82.38) (end 166.6383 82.38) (width 0.25) (layer "F.Cu") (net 2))
 (segment (start 166.6383 82.38) (end 158.0183 91) (width 0.25) (layer "F.Cu") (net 2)))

